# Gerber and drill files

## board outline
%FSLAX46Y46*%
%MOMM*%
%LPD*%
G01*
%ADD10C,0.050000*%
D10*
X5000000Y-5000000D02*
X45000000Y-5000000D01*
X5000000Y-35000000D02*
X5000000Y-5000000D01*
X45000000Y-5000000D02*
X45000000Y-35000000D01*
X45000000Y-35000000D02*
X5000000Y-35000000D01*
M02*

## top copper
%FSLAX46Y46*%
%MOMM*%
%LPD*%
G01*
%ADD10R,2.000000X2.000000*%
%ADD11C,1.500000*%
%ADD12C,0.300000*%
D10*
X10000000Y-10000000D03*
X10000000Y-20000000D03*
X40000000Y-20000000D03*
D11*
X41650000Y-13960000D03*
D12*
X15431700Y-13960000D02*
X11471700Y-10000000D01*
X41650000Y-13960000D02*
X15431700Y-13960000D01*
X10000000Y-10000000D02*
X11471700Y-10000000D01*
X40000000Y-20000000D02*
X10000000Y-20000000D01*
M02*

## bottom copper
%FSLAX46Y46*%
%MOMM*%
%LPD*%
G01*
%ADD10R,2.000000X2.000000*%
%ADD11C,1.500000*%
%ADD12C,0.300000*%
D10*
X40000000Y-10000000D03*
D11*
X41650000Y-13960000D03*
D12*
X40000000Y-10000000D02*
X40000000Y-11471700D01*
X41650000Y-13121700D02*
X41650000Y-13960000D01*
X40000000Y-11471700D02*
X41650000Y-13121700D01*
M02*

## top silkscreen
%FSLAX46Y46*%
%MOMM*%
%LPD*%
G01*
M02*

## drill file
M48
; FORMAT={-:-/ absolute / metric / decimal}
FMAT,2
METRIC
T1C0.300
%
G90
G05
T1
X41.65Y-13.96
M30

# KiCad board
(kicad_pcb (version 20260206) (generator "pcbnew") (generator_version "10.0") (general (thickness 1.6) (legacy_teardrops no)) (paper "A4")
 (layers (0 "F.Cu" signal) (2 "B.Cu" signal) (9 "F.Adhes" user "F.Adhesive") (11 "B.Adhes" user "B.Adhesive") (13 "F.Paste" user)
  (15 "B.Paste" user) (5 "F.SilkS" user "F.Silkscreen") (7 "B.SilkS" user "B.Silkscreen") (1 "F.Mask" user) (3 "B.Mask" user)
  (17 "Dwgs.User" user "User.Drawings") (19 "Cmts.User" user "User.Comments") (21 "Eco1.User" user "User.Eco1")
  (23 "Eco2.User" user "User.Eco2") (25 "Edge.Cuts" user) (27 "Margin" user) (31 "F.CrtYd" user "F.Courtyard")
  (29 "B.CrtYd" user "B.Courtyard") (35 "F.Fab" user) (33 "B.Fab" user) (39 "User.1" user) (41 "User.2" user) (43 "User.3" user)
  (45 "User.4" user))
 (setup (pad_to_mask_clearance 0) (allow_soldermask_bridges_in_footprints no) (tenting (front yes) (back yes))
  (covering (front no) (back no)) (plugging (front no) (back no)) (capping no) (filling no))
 (gr_line (start 5 5) (end 45 5) (stroke (width 0.05) (type default)) (layer "Edge.Cuts"))
 (gr_line (start 5 35) (end 5 5) (stroke (width 0.05) (type default)) (layer "Edge.Cuts"))
 (gr_line (start 45 5) (end 45 35) (stroke (width 0.05) (type default)) (layer "Edge.Cuts"))
 (gr_line (start 45 35) (end 5 35) (stroke (width 0.05) (type default)) (layer "Edge.Cuts"))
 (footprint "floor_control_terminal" (layer "F.Cu") (at 10 10)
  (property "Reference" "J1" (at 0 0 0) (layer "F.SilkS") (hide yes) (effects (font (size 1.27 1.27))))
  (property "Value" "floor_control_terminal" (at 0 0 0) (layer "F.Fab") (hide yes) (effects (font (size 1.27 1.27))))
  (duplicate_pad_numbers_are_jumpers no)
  (pad "1" smd rect (at 0 0) (size 2 2) (layers "F.Cu" "F.Paste" "F.Mask") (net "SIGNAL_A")))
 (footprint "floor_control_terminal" (layer "B.Cu") (at 40 10)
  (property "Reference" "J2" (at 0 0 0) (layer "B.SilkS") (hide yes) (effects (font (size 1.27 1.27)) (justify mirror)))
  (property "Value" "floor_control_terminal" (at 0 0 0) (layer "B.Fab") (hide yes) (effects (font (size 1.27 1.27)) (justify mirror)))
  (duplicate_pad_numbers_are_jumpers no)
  (pad "1" smd rect (at 0 0) (size 2 2) (layers "B.Cu" "B.Paste" "B.Mask") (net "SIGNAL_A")))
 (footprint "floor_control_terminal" (layer "F.Cu") (at 10 20)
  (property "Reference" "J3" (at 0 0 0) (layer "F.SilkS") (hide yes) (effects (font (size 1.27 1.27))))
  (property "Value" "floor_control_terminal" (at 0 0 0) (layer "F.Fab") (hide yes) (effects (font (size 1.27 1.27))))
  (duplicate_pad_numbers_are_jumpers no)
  (pad "1" smd rect (at 0 0) (size 2 2) (layers "F.Cu" "F.Paste" "F.Mask") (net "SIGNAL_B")))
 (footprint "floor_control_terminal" (layer "F.Cu") (at 40 20)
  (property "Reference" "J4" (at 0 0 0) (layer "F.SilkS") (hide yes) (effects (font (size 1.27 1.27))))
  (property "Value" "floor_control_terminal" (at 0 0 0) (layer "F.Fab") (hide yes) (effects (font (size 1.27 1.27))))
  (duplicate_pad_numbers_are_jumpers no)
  (pad "1" smd rect (at 0 0) (size 2 2) (layers "F.Cu" "F.Paste" "F.Mask") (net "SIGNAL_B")))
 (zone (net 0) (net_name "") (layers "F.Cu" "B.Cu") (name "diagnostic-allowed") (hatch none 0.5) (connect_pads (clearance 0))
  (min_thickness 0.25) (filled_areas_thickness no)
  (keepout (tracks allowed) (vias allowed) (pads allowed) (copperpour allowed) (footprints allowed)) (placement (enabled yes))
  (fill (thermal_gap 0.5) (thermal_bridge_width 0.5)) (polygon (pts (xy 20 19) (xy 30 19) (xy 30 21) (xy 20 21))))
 (segment (start 15.4317 13.96) (end 11.4717 10) (width 0.3) (layer "F.Cu") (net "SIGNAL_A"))
 (segment (start 41.65 13.96) (end 15.4317 13.96) (width 0.3) (layer "F.Cu") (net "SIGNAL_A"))
 (segment (start 10 10) (end 11.4717 10) (width 0.3) (layer "F.Cu") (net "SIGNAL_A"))
 (via (at 41.65 13.96) (size 1.5) (drill 0.3) (layers "F.Cu" "B.Cu") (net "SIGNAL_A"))
 (segment (start 40 10) (end 40 11.4717) (width 0.3) (layer "B.Cu") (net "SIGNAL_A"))
 (segment (start 41.65 13.1217) (end 41.65 13.96) (width 0.3) (layer "B.Cu") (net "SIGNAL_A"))
 (segment (start 40 11.4717) (end 41.65 13.1217) (width 0.3) (layer "B.Cu") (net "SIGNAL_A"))
 (segment (start 40 20) (end 10 20) (width 0.3) (layer "F.Cu") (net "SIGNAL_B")))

